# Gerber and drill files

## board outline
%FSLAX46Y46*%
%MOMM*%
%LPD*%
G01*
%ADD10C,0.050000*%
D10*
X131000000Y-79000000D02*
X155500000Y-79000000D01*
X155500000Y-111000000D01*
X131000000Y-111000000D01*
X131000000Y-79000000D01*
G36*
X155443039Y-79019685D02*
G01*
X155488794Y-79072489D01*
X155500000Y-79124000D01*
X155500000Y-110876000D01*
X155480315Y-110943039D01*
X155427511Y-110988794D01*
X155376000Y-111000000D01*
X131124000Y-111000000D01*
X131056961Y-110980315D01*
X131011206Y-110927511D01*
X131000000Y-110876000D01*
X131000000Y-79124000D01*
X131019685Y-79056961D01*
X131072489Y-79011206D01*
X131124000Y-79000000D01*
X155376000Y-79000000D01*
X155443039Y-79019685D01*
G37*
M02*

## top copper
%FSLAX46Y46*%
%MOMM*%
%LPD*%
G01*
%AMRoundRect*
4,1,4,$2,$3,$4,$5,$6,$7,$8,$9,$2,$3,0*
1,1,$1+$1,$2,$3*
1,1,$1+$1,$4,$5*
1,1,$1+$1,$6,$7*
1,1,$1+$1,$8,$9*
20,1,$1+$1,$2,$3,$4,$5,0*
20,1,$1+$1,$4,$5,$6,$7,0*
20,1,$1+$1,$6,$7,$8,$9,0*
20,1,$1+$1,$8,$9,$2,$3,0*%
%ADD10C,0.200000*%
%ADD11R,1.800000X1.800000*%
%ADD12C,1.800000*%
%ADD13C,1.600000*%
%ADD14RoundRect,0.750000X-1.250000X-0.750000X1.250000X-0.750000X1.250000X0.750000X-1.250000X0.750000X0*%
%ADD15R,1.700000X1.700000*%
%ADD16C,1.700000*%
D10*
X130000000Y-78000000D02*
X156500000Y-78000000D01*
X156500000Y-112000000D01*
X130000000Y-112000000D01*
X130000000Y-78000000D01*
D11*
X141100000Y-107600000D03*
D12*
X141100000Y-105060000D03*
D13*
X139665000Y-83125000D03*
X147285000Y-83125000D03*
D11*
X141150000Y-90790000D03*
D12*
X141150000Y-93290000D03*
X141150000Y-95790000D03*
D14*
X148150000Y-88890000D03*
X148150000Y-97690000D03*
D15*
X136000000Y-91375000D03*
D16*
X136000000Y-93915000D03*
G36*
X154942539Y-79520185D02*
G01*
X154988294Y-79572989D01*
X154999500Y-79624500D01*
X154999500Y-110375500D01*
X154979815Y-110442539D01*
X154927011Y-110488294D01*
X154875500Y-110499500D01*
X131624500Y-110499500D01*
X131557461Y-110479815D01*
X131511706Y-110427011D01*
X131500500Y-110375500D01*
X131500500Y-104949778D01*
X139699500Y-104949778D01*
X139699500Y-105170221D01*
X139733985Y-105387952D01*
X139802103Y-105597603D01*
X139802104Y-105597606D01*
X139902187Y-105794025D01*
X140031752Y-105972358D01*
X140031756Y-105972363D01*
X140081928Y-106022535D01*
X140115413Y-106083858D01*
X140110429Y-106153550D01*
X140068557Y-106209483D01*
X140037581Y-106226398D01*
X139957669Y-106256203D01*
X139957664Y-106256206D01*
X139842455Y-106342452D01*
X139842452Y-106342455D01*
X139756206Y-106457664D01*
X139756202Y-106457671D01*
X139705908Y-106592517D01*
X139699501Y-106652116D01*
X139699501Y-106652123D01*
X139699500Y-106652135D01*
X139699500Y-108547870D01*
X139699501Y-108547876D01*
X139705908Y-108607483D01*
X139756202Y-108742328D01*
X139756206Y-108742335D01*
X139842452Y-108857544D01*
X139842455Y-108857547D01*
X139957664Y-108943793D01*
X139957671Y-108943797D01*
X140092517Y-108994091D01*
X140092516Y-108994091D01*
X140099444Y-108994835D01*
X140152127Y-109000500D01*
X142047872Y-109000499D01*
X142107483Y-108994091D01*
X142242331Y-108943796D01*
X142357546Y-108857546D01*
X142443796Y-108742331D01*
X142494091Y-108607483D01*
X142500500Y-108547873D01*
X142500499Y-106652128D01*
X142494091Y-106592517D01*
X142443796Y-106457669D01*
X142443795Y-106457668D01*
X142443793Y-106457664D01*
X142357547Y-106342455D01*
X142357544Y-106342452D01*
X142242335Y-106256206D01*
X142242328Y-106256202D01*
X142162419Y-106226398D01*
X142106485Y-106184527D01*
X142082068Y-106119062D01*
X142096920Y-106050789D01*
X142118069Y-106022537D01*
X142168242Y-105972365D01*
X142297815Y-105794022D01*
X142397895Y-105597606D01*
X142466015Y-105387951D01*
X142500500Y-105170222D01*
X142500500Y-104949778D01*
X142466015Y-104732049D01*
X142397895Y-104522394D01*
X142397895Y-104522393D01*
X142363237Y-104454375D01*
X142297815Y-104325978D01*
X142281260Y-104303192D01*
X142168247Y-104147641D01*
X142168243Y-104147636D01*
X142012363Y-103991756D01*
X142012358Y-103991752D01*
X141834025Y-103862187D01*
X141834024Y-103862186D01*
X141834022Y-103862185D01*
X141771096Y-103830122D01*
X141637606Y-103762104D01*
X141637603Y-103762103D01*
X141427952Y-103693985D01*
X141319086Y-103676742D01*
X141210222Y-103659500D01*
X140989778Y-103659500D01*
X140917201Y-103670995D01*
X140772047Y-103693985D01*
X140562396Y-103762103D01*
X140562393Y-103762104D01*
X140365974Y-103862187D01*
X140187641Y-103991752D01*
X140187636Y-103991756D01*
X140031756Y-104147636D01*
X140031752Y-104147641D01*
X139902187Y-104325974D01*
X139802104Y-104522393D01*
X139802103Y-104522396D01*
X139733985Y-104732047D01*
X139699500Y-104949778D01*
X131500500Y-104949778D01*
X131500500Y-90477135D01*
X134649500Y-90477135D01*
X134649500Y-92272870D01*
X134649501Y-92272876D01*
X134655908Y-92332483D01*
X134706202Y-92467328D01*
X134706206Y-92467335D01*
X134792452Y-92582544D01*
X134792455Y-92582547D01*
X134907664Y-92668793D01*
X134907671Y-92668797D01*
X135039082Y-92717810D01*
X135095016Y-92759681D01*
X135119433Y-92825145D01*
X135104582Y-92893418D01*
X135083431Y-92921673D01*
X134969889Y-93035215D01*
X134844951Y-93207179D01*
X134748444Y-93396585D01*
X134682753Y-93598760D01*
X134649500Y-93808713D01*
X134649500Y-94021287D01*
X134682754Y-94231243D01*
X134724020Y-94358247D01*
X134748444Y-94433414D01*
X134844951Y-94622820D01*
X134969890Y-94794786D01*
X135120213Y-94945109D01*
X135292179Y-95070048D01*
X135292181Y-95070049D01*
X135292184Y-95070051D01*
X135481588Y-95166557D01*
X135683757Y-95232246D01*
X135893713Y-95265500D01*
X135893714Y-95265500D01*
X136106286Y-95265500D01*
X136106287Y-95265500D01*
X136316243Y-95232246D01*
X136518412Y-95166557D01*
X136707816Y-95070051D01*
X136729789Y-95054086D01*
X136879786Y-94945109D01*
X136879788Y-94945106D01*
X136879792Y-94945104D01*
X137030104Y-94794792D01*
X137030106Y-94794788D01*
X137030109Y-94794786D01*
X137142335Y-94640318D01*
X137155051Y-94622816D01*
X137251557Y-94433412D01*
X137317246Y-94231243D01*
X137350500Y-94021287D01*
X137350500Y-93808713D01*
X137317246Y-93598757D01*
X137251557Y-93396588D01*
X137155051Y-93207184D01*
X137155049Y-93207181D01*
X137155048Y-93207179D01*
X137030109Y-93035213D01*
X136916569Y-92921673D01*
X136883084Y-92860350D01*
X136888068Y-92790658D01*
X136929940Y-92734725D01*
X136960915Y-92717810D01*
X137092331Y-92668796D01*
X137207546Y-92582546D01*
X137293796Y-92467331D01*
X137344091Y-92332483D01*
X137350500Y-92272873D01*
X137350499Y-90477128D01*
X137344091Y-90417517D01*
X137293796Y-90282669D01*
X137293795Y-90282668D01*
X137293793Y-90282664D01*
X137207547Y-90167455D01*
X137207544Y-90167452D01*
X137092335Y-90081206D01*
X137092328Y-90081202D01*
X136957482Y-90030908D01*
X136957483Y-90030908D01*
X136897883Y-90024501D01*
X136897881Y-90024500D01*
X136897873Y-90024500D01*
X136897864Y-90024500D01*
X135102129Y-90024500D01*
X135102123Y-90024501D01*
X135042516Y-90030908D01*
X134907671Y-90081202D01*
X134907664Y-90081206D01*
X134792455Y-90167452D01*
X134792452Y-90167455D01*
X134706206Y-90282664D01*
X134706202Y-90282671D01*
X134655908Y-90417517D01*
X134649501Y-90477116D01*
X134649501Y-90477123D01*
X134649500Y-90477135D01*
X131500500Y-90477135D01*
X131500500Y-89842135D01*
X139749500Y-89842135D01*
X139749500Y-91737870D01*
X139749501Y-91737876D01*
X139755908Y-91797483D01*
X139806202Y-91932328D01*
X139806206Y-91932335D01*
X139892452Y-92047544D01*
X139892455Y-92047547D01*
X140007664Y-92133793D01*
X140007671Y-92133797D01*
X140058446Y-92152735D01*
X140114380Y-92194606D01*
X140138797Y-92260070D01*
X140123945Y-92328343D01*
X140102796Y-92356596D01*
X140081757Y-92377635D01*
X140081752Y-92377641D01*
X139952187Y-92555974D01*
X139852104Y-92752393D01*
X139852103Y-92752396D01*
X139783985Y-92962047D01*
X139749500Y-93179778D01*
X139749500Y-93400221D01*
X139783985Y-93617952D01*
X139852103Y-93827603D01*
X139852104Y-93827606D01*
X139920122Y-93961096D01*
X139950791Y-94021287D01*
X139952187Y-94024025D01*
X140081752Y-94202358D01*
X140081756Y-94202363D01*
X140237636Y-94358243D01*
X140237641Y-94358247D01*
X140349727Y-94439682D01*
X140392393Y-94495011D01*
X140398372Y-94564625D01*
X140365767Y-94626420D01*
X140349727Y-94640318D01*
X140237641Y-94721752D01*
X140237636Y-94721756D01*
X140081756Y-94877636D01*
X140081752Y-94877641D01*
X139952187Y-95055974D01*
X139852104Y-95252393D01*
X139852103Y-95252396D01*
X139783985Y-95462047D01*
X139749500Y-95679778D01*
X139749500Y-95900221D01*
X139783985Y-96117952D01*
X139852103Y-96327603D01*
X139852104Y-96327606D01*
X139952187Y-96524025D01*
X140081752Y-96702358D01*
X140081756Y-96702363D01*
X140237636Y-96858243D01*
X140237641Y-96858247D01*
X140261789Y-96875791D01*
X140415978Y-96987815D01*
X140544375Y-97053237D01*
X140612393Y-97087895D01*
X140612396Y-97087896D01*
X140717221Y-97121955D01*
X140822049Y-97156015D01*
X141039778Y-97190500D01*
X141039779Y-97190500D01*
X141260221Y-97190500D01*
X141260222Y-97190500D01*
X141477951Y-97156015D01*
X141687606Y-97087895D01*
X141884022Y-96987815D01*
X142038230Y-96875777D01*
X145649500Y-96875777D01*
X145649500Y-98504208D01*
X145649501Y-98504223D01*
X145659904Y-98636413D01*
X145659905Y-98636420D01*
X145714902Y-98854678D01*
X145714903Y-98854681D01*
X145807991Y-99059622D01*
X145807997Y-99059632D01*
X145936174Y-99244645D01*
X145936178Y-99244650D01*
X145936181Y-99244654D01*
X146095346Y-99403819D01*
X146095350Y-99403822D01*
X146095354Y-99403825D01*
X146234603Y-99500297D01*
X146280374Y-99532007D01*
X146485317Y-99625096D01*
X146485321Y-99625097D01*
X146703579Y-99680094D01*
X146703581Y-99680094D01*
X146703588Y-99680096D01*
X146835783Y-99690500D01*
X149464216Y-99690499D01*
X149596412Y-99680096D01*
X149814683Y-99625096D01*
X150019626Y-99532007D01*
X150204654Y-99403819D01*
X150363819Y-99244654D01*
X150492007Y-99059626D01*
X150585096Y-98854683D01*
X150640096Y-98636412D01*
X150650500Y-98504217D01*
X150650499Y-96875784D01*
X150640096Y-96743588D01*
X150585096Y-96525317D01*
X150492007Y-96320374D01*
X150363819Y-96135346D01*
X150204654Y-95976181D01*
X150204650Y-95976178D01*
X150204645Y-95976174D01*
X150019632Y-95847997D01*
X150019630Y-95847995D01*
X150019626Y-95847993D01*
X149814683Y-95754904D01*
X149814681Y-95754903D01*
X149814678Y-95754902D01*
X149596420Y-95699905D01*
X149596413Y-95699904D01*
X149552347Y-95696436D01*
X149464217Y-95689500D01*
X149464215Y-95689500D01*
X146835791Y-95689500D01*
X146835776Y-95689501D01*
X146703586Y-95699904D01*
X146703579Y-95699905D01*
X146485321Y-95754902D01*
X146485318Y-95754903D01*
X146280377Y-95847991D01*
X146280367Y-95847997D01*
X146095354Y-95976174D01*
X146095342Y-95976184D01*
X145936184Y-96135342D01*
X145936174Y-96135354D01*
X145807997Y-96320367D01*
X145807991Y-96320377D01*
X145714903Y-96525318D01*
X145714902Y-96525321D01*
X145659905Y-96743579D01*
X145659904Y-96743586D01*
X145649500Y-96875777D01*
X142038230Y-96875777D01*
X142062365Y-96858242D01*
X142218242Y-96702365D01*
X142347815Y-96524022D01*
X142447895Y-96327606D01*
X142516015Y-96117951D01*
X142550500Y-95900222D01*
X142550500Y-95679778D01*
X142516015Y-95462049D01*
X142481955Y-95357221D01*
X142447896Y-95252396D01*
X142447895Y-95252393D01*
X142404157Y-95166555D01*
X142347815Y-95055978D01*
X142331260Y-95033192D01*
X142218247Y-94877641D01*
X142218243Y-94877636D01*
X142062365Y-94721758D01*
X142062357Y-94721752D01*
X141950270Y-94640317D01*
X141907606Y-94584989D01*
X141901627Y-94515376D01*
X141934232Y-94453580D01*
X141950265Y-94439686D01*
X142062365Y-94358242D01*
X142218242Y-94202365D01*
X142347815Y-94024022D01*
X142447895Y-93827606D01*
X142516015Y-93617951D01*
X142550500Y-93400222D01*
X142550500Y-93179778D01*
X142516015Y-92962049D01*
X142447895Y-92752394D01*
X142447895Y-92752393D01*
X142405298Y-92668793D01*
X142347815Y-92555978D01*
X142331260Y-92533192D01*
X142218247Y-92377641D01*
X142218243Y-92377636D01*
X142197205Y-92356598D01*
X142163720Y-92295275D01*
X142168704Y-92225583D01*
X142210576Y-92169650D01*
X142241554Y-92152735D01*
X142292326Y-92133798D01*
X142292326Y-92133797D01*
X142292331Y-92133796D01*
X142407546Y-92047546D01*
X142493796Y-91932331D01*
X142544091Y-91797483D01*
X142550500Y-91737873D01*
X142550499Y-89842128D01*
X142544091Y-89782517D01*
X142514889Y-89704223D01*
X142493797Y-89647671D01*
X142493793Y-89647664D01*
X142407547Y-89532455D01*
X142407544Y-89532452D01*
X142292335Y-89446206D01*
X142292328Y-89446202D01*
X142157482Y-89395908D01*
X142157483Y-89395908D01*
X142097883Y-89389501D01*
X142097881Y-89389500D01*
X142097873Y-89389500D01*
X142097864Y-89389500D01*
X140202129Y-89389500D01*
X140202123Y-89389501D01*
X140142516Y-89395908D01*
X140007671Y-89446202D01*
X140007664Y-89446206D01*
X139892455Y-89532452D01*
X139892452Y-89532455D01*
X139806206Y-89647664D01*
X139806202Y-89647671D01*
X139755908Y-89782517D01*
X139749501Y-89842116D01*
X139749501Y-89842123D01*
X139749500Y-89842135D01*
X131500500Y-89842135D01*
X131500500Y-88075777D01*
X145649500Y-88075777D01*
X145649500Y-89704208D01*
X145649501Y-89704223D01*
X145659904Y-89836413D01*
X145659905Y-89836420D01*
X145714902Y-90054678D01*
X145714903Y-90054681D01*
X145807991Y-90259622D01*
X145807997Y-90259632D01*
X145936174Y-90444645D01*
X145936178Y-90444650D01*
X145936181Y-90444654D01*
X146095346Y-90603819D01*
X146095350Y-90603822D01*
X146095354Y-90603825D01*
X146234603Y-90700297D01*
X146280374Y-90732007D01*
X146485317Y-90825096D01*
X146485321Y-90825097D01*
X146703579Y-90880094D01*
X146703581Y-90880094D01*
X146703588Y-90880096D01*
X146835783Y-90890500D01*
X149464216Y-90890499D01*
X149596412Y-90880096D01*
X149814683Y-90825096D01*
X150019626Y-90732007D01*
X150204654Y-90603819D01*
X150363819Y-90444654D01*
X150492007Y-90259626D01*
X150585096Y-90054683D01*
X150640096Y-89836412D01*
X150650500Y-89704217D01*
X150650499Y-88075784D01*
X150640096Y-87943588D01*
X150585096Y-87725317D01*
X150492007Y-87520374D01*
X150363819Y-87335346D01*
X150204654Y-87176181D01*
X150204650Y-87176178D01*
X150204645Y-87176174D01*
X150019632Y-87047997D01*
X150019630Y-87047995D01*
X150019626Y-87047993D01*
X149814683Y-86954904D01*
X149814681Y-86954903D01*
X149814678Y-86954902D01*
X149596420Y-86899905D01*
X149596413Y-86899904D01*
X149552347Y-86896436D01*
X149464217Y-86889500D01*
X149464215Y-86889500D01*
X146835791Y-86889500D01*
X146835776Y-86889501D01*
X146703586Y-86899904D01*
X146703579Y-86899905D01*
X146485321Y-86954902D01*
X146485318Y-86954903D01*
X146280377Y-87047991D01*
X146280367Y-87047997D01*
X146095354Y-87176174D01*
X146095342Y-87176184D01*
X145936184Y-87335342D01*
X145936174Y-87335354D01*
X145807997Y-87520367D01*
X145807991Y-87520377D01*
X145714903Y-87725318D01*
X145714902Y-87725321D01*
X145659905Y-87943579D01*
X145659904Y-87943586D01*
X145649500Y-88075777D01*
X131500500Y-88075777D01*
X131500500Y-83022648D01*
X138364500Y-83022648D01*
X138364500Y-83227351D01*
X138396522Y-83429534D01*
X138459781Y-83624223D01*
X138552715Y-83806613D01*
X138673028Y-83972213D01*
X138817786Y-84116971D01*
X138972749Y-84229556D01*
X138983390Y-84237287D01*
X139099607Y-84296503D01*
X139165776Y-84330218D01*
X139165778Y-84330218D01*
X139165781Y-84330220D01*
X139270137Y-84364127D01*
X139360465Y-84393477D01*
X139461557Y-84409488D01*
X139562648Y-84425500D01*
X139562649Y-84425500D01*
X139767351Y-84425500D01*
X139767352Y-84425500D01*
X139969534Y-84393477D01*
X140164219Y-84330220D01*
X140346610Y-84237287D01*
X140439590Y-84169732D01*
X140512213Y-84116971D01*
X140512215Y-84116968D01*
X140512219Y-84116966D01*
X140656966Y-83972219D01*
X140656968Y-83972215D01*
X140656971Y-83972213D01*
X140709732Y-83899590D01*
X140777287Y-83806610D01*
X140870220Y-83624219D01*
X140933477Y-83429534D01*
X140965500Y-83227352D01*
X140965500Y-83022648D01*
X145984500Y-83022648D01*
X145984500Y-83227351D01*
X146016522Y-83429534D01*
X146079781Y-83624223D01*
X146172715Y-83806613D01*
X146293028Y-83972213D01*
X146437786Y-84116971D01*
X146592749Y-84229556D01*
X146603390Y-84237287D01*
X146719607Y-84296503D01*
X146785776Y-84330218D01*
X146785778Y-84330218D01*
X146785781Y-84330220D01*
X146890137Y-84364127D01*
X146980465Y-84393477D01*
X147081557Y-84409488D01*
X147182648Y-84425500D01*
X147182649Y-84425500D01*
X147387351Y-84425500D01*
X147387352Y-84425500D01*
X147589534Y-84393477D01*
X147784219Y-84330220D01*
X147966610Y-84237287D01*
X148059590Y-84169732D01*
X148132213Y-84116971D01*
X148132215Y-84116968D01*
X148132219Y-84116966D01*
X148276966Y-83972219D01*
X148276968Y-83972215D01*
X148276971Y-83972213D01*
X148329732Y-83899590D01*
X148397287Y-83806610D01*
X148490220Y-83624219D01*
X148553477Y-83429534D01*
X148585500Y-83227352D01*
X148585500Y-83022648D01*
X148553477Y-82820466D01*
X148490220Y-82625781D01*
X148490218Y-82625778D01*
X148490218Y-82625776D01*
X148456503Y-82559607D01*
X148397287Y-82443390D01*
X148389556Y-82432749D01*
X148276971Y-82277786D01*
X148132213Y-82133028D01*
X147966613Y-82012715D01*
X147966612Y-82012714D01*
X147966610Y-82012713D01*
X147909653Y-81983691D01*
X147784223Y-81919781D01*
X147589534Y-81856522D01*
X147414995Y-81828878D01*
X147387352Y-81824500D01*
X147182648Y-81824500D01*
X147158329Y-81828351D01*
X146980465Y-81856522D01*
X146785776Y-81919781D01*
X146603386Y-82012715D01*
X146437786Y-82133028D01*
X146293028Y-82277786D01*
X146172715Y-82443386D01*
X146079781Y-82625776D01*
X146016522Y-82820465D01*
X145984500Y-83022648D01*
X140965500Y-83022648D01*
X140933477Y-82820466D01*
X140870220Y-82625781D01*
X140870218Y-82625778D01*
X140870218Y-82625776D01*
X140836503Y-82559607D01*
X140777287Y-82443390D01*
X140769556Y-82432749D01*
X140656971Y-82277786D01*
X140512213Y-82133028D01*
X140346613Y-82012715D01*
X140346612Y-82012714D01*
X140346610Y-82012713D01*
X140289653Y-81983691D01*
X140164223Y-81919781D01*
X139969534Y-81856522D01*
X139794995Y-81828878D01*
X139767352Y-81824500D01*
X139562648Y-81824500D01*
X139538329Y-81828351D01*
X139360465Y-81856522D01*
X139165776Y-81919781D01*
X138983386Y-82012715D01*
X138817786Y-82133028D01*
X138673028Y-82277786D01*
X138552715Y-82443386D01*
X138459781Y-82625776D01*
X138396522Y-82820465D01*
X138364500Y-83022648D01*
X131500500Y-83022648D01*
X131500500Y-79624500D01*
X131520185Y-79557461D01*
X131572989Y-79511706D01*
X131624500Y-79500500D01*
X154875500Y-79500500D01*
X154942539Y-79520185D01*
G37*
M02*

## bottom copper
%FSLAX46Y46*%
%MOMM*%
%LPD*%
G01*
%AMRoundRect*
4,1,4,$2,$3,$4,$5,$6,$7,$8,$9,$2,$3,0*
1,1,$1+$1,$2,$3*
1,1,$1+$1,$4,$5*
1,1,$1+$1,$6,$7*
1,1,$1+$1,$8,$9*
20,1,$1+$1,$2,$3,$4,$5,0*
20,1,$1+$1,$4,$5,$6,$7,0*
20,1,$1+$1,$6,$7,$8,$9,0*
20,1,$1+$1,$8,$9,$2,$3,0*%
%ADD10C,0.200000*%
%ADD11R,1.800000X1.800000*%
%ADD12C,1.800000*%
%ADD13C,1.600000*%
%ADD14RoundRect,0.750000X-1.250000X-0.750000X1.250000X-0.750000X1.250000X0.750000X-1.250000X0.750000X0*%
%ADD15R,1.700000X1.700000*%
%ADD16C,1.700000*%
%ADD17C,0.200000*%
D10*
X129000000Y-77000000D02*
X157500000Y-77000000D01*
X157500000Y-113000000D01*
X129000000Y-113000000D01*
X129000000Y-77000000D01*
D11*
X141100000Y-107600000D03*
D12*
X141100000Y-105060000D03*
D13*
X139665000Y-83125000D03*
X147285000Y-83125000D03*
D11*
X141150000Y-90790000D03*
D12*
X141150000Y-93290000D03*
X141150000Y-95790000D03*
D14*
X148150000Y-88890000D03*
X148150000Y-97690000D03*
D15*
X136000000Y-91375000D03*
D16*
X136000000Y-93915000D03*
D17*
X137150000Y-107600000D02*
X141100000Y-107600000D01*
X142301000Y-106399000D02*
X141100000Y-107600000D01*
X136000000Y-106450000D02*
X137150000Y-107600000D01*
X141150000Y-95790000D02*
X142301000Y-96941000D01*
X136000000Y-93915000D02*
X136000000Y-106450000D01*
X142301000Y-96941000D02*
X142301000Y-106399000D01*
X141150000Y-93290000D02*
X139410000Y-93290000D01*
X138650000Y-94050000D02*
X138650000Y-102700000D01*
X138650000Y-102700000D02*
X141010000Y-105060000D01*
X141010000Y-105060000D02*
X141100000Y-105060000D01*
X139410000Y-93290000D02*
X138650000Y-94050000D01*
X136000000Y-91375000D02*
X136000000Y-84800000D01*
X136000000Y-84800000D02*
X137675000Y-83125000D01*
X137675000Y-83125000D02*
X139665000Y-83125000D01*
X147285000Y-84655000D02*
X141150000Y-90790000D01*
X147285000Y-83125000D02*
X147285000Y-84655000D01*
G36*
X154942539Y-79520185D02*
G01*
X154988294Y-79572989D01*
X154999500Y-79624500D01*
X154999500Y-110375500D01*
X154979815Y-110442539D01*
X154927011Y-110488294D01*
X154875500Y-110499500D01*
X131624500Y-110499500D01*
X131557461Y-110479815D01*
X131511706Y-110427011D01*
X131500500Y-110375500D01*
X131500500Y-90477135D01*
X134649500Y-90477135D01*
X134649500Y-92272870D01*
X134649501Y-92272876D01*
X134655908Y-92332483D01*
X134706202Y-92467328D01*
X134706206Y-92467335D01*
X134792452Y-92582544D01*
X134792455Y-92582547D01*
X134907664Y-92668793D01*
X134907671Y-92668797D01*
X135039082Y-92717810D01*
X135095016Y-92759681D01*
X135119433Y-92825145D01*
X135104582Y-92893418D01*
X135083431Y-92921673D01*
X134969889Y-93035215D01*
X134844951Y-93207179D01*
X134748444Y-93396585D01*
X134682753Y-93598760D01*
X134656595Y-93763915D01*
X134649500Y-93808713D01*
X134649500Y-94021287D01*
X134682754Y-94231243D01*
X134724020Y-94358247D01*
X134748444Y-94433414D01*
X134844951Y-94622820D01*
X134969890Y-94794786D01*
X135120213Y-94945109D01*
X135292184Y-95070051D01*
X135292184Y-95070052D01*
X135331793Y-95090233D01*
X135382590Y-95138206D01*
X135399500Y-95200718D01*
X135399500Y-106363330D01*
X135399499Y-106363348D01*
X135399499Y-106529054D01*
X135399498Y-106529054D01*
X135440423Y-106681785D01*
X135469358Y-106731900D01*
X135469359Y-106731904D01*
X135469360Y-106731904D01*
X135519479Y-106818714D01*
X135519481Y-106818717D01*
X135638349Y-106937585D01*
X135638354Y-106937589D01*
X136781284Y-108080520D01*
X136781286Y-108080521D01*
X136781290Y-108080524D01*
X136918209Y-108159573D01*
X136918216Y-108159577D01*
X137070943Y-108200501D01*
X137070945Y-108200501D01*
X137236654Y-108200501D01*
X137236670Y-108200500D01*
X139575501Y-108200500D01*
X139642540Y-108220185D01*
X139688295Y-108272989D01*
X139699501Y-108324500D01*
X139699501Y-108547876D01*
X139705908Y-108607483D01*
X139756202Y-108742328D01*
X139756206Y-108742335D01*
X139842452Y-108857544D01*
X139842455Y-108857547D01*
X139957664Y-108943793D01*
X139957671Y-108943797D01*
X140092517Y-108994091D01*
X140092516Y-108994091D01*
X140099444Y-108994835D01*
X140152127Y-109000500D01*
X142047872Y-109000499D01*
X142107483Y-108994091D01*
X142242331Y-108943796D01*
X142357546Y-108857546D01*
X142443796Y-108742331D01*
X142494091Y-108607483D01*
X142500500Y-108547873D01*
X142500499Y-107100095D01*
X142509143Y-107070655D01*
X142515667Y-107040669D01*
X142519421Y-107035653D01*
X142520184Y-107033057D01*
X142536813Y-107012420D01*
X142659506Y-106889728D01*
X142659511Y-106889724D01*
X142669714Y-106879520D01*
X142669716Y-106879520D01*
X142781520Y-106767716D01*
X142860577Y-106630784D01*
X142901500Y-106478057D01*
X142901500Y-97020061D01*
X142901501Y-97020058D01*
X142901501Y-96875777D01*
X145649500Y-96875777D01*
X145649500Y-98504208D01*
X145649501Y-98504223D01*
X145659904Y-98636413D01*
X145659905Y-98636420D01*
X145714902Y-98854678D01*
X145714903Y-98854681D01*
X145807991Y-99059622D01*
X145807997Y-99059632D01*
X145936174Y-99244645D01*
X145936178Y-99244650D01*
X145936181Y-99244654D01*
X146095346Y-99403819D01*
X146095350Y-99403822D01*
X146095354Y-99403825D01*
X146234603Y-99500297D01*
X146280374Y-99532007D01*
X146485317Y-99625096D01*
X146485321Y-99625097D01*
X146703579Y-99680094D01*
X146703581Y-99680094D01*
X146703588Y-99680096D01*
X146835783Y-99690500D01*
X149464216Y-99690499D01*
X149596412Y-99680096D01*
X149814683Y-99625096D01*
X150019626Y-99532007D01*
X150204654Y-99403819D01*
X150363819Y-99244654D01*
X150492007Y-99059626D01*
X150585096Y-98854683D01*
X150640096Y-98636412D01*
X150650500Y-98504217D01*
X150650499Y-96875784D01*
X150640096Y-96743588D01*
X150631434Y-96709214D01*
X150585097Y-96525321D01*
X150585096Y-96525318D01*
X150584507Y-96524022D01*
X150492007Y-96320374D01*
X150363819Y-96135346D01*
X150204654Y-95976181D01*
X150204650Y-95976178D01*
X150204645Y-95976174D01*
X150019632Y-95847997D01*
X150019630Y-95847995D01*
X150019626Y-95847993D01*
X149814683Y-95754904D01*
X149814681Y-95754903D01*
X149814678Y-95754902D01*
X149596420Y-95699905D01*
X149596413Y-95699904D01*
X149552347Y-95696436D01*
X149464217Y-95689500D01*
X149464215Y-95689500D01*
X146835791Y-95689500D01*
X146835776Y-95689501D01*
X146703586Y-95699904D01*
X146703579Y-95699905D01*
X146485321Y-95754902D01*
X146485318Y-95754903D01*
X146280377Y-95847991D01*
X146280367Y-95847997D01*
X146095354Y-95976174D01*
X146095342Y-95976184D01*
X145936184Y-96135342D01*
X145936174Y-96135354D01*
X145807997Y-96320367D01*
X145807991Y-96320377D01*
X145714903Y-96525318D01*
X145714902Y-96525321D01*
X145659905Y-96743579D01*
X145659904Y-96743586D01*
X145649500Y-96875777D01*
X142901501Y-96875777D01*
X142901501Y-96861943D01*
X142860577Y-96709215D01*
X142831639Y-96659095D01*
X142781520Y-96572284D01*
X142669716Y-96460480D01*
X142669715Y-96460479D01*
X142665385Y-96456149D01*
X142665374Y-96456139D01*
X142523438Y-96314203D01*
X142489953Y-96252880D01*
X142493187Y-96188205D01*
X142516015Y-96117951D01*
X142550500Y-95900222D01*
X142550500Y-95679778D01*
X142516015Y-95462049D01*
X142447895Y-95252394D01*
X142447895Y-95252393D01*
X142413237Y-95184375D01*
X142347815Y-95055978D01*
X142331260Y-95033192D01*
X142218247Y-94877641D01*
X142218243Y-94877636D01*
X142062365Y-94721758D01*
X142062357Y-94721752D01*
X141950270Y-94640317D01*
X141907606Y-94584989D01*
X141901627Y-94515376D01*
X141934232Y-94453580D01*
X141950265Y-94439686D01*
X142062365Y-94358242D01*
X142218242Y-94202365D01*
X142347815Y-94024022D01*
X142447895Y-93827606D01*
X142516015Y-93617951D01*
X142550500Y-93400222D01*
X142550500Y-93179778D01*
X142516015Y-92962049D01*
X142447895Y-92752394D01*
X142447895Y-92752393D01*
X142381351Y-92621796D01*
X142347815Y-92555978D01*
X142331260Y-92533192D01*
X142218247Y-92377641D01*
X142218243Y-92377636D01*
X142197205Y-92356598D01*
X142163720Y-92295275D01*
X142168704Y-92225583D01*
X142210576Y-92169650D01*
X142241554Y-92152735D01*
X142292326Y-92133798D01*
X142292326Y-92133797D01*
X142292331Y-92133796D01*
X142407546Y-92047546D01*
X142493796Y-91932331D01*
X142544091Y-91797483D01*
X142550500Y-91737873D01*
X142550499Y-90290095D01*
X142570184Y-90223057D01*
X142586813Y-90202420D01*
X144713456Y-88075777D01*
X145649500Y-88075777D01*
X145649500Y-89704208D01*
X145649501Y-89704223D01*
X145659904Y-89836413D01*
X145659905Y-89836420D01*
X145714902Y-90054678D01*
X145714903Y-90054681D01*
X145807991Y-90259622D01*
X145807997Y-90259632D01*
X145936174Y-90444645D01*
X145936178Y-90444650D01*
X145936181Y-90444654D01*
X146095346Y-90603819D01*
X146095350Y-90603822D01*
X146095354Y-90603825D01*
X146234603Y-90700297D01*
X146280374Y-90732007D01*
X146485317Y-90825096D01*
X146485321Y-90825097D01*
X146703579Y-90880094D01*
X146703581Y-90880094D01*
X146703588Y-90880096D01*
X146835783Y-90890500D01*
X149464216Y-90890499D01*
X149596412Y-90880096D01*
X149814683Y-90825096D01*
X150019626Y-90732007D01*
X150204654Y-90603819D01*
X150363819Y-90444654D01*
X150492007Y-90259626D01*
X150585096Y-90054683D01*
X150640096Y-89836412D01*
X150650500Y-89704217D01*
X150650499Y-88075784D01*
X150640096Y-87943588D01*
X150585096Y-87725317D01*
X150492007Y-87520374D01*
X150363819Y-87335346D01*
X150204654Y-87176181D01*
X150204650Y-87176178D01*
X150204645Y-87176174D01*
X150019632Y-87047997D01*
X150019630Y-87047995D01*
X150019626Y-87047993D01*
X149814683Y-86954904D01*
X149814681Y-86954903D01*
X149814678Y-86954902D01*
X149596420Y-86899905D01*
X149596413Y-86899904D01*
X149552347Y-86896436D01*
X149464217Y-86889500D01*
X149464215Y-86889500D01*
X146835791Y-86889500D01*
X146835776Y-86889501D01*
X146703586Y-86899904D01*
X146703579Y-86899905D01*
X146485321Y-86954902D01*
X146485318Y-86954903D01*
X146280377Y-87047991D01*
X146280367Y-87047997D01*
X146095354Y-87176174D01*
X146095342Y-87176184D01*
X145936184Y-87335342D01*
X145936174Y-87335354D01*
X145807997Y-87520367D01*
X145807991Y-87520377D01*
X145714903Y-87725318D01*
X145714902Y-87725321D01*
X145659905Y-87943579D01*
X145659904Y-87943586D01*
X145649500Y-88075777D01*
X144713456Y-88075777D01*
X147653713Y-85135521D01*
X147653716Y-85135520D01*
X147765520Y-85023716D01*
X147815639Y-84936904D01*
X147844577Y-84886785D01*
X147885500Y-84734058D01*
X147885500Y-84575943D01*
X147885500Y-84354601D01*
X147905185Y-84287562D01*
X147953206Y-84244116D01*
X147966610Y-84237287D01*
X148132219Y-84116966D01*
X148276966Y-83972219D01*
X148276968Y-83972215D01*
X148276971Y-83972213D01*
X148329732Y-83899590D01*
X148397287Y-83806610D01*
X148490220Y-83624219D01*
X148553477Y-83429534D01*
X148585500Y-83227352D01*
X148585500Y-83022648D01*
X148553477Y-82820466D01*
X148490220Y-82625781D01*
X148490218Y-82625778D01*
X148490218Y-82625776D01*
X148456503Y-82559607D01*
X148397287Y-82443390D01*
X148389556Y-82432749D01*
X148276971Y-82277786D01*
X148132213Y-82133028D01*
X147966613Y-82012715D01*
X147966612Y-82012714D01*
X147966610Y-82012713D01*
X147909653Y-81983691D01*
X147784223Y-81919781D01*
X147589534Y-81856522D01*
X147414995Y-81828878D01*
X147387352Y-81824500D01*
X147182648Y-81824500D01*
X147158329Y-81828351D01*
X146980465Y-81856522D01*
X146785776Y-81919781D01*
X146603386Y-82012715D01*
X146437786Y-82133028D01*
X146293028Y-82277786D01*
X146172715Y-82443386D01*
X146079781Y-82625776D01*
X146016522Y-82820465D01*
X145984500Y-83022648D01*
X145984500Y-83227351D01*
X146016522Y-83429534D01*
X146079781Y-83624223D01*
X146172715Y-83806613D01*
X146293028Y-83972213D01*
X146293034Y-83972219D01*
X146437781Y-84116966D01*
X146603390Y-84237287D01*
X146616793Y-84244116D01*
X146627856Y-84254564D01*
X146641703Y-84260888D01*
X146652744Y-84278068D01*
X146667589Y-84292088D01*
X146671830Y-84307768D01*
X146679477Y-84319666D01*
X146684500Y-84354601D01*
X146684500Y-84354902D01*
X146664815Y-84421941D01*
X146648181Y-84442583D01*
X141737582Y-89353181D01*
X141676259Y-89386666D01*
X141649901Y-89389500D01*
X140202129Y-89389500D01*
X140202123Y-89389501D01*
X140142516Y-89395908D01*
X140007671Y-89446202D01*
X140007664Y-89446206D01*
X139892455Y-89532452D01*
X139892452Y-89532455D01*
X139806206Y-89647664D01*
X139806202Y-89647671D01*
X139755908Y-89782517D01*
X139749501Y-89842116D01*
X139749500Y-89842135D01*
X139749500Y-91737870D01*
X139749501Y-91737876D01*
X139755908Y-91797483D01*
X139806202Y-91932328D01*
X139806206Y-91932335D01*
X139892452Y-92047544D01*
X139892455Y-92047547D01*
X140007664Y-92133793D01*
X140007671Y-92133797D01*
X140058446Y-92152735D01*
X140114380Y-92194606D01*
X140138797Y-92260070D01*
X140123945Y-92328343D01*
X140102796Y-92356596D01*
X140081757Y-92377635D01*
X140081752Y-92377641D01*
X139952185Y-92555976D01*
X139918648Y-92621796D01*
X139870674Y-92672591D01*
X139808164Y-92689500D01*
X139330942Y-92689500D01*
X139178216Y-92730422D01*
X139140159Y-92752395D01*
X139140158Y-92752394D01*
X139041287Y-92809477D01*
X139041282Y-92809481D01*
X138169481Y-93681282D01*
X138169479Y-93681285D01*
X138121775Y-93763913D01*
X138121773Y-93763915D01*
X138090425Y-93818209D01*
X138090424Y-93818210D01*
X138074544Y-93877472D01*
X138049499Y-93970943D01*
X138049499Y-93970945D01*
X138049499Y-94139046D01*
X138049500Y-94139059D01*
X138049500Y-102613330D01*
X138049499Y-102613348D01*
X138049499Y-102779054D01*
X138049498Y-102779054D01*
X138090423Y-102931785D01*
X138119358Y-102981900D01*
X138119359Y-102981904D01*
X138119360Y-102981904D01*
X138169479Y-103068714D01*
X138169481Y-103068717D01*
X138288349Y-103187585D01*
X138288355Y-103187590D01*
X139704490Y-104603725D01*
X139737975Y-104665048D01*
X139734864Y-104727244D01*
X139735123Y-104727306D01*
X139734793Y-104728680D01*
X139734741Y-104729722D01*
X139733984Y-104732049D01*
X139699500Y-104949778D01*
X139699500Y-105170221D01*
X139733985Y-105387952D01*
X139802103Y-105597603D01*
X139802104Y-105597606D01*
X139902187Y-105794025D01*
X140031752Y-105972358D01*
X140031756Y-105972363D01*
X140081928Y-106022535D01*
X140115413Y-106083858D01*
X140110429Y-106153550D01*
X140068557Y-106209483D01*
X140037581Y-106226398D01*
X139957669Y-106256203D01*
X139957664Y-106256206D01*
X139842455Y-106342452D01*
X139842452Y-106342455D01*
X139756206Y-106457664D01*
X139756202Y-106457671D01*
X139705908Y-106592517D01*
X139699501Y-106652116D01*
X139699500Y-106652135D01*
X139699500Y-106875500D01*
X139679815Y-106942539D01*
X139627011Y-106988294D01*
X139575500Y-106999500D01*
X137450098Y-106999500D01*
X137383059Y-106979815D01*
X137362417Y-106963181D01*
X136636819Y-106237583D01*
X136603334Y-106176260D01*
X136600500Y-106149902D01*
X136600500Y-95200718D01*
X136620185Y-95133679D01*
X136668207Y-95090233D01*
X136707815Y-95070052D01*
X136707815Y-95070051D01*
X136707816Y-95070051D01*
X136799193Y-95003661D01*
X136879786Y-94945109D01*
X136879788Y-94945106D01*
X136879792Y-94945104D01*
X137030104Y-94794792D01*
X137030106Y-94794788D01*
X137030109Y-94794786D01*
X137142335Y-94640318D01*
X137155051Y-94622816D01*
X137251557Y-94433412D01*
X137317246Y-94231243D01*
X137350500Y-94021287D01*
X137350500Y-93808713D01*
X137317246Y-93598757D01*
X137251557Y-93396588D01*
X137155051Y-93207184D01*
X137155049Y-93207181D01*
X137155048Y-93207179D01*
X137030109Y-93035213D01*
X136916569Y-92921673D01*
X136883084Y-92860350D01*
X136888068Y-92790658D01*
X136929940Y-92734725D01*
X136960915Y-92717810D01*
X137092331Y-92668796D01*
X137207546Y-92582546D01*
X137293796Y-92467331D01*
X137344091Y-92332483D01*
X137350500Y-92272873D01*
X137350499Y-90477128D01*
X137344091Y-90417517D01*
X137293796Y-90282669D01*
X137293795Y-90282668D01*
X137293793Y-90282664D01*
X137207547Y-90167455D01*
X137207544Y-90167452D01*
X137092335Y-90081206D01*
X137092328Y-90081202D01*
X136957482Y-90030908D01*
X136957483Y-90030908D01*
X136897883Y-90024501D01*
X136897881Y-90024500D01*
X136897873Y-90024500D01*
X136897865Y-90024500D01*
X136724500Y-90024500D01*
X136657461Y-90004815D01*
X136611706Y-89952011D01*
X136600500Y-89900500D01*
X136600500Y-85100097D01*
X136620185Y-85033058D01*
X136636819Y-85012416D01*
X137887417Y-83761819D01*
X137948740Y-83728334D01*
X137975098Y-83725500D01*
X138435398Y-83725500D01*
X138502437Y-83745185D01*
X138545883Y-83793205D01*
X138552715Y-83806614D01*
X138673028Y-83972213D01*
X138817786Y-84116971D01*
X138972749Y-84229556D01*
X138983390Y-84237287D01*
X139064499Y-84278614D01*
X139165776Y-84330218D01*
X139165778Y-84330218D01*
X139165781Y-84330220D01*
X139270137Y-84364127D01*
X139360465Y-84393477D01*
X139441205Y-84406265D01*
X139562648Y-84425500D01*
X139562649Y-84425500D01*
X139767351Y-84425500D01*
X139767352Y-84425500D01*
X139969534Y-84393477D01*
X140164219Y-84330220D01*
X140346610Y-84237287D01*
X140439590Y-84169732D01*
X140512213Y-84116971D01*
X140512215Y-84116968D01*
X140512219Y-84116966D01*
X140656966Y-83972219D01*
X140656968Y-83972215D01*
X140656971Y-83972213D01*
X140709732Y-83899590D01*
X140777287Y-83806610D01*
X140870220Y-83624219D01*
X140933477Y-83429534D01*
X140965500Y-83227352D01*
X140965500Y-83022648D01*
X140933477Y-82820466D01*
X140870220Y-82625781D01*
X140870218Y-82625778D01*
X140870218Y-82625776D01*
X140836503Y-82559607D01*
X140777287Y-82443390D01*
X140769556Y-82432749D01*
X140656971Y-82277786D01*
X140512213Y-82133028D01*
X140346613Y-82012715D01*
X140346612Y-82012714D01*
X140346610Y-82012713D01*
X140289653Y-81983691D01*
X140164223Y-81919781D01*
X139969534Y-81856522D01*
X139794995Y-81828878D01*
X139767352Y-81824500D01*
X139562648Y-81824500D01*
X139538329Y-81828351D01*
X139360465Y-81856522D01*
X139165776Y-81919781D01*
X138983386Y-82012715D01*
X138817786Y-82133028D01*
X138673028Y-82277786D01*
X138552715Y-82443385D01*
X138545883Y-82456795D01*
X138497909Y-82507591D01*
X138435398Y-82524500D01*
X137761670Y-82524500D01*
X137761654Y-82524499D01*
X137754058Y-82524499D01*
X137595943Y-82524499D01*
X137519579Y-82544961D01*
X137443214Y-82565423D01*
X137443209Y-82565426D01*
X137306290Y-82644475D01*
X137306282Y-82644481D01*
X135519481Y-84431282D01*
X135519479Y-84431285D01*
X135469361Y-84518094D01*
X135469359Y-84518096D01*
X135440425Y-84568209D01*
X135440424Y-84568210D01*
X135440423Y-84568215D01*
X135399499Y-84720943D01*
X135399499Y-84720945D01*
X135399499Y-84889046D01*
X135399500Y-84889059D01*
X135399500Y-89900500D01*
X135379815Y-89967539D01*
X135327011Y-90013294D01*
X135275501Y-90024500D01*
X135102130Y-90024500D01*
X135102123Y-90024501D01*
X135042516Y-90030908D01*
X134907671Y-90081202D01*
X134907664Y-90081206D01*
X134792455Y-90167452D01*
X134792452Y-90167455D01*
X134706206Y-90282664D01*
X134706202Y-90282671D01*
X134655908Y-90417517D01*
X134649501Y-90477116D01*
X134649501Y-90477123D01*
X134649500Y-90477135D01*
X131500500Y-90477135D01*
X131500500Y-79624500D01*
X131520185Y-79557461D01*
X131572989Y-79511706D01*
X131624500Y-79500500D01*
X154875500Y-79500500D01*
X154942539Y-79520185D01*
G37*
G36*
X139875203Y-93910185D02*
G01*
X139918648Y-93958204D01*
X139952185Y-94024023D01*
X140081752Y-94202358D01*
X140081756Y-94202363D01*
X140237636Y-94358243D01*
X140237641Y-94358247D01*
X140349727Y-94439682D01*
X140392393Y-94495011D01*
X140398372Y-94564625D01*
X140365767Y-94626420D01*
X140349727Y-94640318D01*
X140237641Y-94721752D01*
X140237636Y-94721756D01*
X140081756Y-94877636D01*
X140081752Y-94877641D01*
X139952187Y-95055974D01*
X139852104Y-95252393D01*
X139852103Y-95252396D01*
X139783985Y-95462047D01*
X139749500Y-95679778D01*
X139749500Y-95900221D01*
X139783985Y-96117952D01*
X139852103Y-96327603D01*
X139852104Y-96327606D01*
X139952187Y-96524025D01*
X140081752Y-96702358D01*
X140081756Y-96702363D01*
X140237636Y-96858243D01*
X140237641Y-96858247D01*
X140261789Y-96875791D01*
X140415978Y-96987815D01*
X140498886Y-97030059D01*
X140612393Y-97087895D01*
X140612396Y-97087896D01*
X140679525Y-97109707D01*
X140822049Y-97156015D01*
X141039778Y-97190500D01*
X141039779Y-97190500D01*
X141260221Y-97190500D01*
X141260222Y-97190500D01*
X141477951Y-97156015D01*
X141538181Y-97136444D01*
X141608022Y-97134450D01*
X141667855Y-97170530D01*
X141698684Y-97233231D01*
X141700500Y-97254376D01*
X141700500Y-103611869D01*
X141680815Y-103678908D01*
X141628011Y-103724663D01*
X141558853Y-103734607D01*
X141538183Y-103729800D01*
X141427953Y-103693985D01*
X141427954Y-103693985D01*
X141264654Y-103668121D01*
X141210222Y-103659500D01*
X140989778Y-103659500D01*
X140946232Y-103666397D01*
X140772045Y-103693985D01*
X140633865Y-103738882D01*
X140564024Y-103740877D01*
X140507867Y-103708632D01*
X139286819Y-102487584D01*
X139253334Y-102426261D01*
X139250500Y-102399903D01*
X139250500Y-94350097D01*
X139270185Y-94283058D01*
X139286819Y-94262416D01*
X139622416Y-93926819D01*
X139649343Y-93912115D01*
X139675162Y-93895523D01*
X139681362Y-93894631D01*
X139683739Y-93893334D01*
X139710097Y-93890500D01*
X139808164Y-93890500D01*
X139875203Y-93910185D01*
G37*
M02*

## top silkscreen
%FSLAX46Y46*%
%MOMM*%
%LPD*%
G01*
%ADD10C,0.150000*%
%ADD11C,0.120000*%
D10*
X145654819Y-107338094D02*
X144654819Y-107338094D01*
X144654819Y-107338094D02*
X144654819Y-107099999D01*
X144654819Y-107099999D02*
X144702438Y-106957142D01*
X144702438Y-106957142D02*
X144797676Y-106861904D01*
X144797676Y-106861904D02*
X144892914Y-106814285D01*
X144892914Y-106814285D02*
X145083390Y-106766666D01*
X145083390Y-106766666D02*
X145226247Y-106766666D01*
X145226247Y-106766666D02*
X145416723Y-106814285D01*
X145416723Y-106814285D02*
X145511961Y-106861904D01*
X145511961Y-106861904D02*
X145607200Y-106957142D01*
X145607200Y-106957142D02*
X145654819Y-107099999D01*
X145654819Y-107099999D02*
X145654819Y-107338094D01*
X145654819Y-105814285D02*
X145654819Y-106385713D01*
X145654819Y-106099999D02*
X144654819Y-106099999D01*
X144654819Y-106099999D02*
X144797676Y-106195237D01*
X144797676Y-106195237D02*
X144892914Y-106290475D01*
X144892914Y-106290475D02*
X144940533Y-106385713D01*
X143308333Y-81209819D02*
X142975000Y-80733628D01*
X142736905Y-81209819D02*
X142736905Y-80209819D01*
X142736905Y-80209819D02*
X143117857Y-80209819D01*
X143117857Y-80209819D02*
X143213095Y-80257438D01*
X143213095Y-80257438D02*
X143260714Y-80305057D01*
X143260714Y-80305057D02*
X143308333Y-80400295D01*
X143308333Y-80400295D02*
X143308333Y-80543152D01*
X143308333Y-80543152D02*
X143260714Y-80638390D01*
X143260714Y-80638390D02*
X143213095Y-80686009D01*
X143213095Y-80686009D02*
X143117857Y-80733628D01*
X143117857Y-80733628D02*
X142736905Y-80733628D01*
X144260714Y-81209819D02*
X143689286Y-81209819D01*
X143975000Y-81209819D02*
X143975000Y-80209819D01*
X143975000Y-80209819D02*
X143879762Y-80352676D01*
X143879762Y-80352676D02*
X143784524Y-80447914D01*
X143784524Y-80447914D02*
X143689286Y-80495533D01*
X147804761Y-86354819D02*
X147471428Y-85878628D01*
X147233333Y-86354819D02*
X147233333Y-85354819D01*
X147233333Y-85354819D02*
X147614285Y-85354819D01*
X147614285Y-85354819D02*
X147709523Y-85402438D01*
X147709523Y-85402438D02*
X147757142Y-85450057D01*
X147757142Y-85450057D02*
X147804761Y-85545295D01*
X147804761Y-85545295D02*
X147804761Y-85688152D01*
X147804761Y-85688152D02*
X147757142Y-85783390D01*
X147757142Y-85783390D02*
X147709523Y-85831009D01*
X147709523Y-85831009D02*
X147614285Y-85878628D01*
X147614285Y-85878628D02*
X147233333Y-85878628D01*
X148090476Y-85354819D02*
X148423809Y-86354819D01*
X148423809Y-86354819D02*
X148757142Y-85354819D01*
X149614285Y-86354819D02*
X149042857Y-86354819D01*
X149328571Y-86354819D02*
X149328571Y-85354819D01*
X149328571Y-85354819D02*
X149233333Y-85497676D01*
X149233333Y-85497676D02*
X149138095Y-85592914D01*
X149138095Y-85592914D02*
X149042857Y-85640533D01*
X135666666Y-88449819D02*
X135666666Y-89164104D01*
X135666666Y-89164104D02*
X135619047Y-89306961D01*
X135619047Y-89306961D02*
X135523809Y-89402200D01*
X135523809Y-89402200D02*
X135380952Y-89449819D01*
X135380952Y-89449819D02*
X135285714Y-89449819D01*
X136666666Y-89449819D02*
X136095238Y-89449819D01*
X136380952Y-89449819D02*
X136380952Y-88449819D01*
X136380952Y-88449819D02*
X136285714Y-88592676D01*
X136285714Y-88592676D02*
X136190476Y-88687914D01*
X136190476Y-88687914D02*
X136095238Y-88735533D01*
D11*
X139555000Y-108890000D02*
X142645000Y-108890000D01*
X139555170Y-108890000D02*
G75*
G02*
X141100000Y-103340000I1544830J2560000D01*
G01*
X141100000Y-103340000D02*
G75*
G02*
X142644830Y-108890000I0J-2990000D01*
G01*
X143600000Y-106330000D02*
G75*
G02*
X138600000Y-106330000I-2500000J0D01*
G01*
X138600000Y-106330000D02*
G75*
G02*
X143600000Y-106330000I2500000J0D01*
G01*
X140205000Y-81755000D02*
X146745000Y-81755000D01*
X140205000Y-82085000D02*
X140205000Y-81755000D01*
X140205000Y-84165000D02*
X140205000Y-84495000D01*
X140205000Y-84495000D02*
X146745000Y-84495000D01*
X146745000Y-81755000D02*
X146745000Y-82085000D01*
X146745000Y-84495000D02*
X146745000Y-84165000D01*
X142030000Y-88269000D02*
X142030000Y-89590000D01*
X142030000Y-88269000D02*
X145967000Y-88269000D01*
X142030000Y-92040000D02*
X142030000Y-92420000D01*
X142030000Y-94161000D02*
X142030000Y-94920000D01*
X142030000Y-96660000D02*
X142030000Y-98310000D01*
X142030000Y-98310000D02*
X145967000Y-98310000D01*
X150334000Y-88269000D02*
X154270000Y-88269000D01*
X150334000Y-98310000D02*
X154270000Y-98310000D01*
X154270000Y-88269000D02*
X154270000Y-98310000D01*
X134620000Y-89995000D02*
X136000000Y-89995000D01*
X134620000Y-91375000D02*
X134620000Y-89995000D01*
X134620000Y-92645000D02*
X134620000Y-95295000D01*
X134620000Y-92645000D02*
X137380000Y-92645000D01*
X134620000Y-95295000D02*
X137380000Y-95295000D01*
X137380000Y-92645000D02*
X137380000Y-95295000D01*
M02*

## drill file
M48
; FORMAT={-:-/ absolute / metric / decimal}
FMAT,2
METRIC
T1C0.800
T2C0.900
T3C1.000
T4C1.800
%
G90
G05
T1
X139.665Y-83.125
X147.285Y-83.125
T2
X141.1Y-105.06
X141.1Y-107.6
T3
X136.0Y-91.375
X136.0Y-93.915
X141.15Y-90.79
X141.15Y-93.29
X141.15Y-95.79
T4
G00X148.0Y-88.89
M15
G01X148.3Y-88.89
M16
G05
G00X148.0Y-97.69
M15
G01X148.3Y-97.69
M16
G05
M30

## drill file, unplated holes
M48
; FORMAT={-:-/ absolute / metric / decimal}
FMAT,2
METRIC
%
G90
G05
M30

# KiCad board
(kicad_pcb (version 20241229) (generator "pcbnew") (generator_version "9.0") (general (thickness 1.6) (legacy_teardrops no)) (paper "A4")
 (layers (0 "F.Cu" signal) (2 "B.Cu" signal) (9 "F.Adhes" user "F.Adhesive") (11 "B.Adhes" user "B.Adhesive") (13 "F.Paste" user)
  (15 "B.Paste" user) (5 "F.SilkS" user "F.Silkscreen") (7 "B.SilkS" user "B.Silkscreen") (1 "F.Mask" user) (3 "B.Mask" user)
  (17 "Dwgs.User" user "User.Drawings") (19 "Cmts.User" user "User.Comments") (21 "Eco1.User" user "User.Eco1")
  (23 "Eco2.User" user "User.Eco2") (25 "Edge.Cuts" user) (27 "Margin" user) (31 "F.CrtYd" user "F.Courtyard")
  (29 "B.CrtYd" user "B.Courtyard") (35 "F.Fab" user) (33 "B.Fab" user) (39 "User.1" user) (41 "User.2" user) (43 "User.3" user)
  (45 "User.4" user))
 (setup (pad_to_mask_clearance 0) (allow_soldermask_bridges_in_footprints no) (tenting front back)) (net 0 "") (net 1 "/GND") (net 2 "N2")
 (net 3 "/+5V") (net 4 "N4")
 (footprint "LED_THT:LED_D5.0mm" (layer "F.Cu") (at 141.1 107.6 90)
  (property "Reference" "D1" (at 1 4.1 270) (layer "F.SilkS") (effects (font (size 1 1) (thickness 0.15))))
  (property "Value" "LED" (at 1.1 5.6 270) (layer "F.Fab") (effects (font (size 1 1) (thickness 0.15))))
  (fp_line (start -1.29 -1.545) (end -1.29 1.545) (stroke (width 0.12) (type solid)) (layer "F.SilkS"))
  (fp_arc (start -1.29 -1.54483) (mid 2.071779 -2.880495) (end 4.26 0) (stroke (width 0.12) (type solid)) (layer "F.SilkS"))
  (fp_arc (start 4.26 0) (mid 2.071779 2.880495) (end -1.29 1.54483) (stroke (width 0.12) (type solid)) (layer "F.SilkS"))
  (fp_circle (center 1.27 0) (end 3.77 0) (stroke (width 0.12) (type solid)) (fill no) (layer "F.SilkS"))
  (pad "1" thru_hole rect (at 0 0 90) (size 1.8 1.8) (drill 0.9) (layers "*.Cu" "*.Mask") (remove_unused_layers no) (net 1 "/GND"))
  (pad "2" thru_hole circle (at 2.54 0 90) (size 1.8 1.8) (drill 0.9) (layers "*.Cu" "*.Mask") (remove_unused_layers no) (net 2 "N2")))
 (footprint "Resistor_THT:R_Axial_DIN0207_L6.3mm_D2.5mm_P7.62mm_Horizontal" (layer "F.Cu") (at 139.665 83.125)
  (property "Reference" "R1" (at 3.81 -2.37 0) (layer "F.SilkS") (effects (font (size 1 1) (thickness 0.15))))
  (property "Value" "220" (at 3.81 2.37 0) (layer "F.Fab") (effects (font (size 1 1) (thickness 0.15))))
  (fp_line (start 0.54 -1.37) (end 7.08 -1.37) (stroke (width 0.12) (type solid)) (layer "F.SilkS"))
  (fp_line (start 0.54 -1.04) (end 0.54 -1.37) (stroke (width 0.12) (type solid)) (layer "F.SilkS"))
  (fp_line (start 0.54 1.04) (end 0.54 1.37) (stroke (width 0.12) (type solid)) (layer "F.SilkS"))
  (fp_line (start 0.54 1.37) (end 7.08 1.37) (stroke (width 0.12) (type solid)) (layer "F.SilkS"))
  (fp_line (start 7.08 -1.37) (end 7.08 -1.04) (stroke (width 0.12) (type solid)) (layer "F.SilkS"))
  (fp_line (start 7.08 1.37) (end 7.08 1.04) (stroke (width 0.12) (type solid)) (layer "F.SilkS"))
  (pad "1" thru_hole circle (at 0 0) (size 1.6 1.6) (drill 0.8) (layers "*.Cu" "*.Mask") (remove_unused_layers no) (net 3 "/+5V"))
  (pad "2" thru_hole circle (at 7.62 0) (size 1.6 1.6) (drill 0.8) (layers "*.Cu" "*.Mask") (remove_unused_layers no) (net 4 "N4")))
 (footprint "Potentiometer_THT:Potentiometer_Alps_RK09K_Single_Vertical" (layer "F.Cu") (at 141.15 90.79)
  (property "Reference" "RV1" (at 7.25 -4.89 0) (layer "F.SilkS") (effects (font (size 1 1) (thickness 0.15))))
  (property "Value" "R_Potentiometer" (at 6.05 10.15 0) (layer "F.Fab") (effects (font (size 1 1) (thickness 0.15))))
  (fp_line (start 0.88 -2.521) (end 0.88 -1.2) (stroke (width 0.12) (type solid)) (layer "F.SilkS"))
  (fp_line (start 0.88 -2.521) (end 4.817 -2.521) (stroke (width 0.12) (type solid)) (layer "F.SilkS"))
  (fp_line (start 0.88 1.25) (end 0.88 1.63) (stroke (width 0.12) (type solid)) (layer "F.SilkS"))
  (fp_line (start 0.88 3.371) (end 0.88 4.13) (stroke (width 0.12) (type solid)) (layer "F.SilkS"))
  (fp_line (start 0.88 5.87) (end 0.88 7.52) (stroke (width 0.12) (type solid)) (layer "F.SilkS"))
  (fp_line (start 0.88 7.52) (end 4.817 7.52) (stroke (width 0.12) (type solid)) (layer "F.SilkS"))
  (fp_line (start 9.184 -2.521) (end 13.12 -2.521) (stroke (width 0.12) (type solid)) (layer "F.SilkS"))
  (fp_line (start 9.184 7.52) (end 13.12 7.52) (stroke (width 0.12) (type solid)) (layer "F.SilkS"))
  (fp_line (start 13.12 -2.521) (end 13.12 7.52) (stroke (width 0.12) (type solid)) (layer "F.SilkS"))
  (pad "1" thru_hole rect (at 0 0) (size 1.8 1.8) (drill 1) (layers "*.Cu" "*.Mask") (remove_unused_layers no) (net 4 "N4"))
  (pad "2" thru_hole circle (at 0 2.5) (size 1.8 1.8) (drill 1) (layers "*.Cu" "*.Mask") (remove_unused_layers no) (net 2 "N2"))
  (pad "3" thru_hole circle (at 0 5) (size 1.8 1.8) (drill 1) (layers "*.Cu" "*.Mask") (remove_unused_layers no) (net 1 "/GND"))
  (pad "MP" thru_hole roundrect (at 7 -1.9) (size 4 3) (drill oval 2.1 1.8) (layers "*.Cu" "*.Mask") (remove_unused_layers no)
   (roundrect_rratio 0.25))
  (pad "MP" thru_hole roundrect (at 7 6.9) (size 4 3) (drill oval 2.1 1.8) (layers "*.Cu" "*.Mask") (remove_unused_layers no)
   (roundrect_rratio 0.25)))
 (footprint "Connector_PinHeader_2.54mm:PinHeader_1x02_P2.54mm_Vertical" (layer "F.Cu") (at 136 91.375)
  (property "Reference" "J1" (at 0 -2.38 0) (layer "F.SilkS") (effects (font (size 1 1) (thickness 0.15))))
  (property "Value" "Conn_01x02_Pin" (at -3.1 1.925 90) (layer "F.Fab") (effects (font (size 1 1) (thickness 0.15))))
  (fp_line (start -1.38 -1.38) (end 0 -1.38) (stroke (width 0.12) (type solid)) (layer "F.SilkS"))
  (fp_line (start -1.38 0) (end -1.38 -1.38) (stroke (width 0.12) (type solid)) (layer "F.SilkS"))
  (fp_line (start -1.38 1.27) (end -1.38 3.92) (stroke (width 0.12) (type solid)) (layer "F.SilkS"))
  (fp_line (start -1.38 1.27) (end 1.38 1.27) (stroke (width 0.12) (type solid)) (layer "F.SilkS"))
  (fp_line (start -1.38 3.92) (end 1.38 3.92) (stroke (width 0.12) (type solid)) (layer "F.SilkS"))
  (fp_line (start 1.38 1.27) (end 1.38 3.92) (stroke (width 0.12) (type solid)) (layer "F.SilkS"))
  (pad "1" thru_hole rect (at 0 0) (size 1.7 1.7) (drill 1) (layers "*.Cu" "*.Mask") (remove_unused_layers no) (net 3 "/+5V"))
  (pad "2" thru_hole circle (at 0 2.54) (size 1.7 1.7) (drill 1) (layers "*.Cu" "*.Mask") (remove_unused_layers no) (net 1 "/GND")))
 (gr_rect (start 130 78) (end 156.5 112) (stroke (width 0.2) (type default)) (fill no) (layer "F.Cu"))
 (gr_rect (start 129 77) (end 157.5 113) (stroke (width 0.2) (type default)) (fill no) (layer "B.Cu"))
 (gr_rect (start 131 79) (end 155.5 111) (stroke (width 0.05) (type default)) (fill no) (layer "Edge.Cuts"))
 (segment (start 137.15 107.6) (end 141.1 107.6) (width 0.2) (layer "B.Cu") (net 1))
 (segment (start 142.301 106.399) (end 141.1 107.6) (width 0.2) (layer "B.Cu") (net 1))
 (segment (start 136 106.45) (end 137.15 107.6) (width 0.2) (layer "B.Cu") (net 1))
 (segment (start 141.15 95.79) (end 142.301 96.941) (width 0.2) (layer "B.Cu") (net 1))
 (segment (start 136 93.915) (end 136 106.45) (width 0.2) (layer "B.Cu") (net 1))
 (segment (start 142.301 96.941) (end 142.301 106.399) (width 0.2) (layer "B.Cu") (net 1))
 (segment (start 141.15 93.29) (end 139.41 93.29) (width 0.2) (layer "B.Cu") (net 2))
 (segment (start 138.65 94.05) (end 138.65 102.7) (width 0.2) (layer "B.Cu") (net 2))
 (segment (start 138.65 102.7) (end 141.01 105.06) (width 0.2) (layer "B.Cu") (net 2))
 (segment (start 141.01 105.06) (end 141.1 105.06) (width 0.2) (layer "B.Cu") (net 2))
 (segment (start 139.41 93.29) (end 138.65 94.05) (width 0.2) (layer "B.Cu") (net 2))
 (segment (start 136 91.375) (end 136 84.8) (width 0.2) (layer "B.Cu") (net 3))
 (segment (start 136 84.8) (end 137.675 83.125) (width 0.2) (layer "B.Cu") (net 3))
 (segment (start 137.675 83.125) (end 139.665 83.125) (width 0.2) (layer "B.Cu") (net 3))
 (segment (start 147.285 84.655) (end 141.15 90.79) (width 0.2) (layer "B.Cu") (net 4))
 (segment (start 147.285 83.125) (end 147.285 84.655) (width 0.2) (layer "B.Cu") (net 4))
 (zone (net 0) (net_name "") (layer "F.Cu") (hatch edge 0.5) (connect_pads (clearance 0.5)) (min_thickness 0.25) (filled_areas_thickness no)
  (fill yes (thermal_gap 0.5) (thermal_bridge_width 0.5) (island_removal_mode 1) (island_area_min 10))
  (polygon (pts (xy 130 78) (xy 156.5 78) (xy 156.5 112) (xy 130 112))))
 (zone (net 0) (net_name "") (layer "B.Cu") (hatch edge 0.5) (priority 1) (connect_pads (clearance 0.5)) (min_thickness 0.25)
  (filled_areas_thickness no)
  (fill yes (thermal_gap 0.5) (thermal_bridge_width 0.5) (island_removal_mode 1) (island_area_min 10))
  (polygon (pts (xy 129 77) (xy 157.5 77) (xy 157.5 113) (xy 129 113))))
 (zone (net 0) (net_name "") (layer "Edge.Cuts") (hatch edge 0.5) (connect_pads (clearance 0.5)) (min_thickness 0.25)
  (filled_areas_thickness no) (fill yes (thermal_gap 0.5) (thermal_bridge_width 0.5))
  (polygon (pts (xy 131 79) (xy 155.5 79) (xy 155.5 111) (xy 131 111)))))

